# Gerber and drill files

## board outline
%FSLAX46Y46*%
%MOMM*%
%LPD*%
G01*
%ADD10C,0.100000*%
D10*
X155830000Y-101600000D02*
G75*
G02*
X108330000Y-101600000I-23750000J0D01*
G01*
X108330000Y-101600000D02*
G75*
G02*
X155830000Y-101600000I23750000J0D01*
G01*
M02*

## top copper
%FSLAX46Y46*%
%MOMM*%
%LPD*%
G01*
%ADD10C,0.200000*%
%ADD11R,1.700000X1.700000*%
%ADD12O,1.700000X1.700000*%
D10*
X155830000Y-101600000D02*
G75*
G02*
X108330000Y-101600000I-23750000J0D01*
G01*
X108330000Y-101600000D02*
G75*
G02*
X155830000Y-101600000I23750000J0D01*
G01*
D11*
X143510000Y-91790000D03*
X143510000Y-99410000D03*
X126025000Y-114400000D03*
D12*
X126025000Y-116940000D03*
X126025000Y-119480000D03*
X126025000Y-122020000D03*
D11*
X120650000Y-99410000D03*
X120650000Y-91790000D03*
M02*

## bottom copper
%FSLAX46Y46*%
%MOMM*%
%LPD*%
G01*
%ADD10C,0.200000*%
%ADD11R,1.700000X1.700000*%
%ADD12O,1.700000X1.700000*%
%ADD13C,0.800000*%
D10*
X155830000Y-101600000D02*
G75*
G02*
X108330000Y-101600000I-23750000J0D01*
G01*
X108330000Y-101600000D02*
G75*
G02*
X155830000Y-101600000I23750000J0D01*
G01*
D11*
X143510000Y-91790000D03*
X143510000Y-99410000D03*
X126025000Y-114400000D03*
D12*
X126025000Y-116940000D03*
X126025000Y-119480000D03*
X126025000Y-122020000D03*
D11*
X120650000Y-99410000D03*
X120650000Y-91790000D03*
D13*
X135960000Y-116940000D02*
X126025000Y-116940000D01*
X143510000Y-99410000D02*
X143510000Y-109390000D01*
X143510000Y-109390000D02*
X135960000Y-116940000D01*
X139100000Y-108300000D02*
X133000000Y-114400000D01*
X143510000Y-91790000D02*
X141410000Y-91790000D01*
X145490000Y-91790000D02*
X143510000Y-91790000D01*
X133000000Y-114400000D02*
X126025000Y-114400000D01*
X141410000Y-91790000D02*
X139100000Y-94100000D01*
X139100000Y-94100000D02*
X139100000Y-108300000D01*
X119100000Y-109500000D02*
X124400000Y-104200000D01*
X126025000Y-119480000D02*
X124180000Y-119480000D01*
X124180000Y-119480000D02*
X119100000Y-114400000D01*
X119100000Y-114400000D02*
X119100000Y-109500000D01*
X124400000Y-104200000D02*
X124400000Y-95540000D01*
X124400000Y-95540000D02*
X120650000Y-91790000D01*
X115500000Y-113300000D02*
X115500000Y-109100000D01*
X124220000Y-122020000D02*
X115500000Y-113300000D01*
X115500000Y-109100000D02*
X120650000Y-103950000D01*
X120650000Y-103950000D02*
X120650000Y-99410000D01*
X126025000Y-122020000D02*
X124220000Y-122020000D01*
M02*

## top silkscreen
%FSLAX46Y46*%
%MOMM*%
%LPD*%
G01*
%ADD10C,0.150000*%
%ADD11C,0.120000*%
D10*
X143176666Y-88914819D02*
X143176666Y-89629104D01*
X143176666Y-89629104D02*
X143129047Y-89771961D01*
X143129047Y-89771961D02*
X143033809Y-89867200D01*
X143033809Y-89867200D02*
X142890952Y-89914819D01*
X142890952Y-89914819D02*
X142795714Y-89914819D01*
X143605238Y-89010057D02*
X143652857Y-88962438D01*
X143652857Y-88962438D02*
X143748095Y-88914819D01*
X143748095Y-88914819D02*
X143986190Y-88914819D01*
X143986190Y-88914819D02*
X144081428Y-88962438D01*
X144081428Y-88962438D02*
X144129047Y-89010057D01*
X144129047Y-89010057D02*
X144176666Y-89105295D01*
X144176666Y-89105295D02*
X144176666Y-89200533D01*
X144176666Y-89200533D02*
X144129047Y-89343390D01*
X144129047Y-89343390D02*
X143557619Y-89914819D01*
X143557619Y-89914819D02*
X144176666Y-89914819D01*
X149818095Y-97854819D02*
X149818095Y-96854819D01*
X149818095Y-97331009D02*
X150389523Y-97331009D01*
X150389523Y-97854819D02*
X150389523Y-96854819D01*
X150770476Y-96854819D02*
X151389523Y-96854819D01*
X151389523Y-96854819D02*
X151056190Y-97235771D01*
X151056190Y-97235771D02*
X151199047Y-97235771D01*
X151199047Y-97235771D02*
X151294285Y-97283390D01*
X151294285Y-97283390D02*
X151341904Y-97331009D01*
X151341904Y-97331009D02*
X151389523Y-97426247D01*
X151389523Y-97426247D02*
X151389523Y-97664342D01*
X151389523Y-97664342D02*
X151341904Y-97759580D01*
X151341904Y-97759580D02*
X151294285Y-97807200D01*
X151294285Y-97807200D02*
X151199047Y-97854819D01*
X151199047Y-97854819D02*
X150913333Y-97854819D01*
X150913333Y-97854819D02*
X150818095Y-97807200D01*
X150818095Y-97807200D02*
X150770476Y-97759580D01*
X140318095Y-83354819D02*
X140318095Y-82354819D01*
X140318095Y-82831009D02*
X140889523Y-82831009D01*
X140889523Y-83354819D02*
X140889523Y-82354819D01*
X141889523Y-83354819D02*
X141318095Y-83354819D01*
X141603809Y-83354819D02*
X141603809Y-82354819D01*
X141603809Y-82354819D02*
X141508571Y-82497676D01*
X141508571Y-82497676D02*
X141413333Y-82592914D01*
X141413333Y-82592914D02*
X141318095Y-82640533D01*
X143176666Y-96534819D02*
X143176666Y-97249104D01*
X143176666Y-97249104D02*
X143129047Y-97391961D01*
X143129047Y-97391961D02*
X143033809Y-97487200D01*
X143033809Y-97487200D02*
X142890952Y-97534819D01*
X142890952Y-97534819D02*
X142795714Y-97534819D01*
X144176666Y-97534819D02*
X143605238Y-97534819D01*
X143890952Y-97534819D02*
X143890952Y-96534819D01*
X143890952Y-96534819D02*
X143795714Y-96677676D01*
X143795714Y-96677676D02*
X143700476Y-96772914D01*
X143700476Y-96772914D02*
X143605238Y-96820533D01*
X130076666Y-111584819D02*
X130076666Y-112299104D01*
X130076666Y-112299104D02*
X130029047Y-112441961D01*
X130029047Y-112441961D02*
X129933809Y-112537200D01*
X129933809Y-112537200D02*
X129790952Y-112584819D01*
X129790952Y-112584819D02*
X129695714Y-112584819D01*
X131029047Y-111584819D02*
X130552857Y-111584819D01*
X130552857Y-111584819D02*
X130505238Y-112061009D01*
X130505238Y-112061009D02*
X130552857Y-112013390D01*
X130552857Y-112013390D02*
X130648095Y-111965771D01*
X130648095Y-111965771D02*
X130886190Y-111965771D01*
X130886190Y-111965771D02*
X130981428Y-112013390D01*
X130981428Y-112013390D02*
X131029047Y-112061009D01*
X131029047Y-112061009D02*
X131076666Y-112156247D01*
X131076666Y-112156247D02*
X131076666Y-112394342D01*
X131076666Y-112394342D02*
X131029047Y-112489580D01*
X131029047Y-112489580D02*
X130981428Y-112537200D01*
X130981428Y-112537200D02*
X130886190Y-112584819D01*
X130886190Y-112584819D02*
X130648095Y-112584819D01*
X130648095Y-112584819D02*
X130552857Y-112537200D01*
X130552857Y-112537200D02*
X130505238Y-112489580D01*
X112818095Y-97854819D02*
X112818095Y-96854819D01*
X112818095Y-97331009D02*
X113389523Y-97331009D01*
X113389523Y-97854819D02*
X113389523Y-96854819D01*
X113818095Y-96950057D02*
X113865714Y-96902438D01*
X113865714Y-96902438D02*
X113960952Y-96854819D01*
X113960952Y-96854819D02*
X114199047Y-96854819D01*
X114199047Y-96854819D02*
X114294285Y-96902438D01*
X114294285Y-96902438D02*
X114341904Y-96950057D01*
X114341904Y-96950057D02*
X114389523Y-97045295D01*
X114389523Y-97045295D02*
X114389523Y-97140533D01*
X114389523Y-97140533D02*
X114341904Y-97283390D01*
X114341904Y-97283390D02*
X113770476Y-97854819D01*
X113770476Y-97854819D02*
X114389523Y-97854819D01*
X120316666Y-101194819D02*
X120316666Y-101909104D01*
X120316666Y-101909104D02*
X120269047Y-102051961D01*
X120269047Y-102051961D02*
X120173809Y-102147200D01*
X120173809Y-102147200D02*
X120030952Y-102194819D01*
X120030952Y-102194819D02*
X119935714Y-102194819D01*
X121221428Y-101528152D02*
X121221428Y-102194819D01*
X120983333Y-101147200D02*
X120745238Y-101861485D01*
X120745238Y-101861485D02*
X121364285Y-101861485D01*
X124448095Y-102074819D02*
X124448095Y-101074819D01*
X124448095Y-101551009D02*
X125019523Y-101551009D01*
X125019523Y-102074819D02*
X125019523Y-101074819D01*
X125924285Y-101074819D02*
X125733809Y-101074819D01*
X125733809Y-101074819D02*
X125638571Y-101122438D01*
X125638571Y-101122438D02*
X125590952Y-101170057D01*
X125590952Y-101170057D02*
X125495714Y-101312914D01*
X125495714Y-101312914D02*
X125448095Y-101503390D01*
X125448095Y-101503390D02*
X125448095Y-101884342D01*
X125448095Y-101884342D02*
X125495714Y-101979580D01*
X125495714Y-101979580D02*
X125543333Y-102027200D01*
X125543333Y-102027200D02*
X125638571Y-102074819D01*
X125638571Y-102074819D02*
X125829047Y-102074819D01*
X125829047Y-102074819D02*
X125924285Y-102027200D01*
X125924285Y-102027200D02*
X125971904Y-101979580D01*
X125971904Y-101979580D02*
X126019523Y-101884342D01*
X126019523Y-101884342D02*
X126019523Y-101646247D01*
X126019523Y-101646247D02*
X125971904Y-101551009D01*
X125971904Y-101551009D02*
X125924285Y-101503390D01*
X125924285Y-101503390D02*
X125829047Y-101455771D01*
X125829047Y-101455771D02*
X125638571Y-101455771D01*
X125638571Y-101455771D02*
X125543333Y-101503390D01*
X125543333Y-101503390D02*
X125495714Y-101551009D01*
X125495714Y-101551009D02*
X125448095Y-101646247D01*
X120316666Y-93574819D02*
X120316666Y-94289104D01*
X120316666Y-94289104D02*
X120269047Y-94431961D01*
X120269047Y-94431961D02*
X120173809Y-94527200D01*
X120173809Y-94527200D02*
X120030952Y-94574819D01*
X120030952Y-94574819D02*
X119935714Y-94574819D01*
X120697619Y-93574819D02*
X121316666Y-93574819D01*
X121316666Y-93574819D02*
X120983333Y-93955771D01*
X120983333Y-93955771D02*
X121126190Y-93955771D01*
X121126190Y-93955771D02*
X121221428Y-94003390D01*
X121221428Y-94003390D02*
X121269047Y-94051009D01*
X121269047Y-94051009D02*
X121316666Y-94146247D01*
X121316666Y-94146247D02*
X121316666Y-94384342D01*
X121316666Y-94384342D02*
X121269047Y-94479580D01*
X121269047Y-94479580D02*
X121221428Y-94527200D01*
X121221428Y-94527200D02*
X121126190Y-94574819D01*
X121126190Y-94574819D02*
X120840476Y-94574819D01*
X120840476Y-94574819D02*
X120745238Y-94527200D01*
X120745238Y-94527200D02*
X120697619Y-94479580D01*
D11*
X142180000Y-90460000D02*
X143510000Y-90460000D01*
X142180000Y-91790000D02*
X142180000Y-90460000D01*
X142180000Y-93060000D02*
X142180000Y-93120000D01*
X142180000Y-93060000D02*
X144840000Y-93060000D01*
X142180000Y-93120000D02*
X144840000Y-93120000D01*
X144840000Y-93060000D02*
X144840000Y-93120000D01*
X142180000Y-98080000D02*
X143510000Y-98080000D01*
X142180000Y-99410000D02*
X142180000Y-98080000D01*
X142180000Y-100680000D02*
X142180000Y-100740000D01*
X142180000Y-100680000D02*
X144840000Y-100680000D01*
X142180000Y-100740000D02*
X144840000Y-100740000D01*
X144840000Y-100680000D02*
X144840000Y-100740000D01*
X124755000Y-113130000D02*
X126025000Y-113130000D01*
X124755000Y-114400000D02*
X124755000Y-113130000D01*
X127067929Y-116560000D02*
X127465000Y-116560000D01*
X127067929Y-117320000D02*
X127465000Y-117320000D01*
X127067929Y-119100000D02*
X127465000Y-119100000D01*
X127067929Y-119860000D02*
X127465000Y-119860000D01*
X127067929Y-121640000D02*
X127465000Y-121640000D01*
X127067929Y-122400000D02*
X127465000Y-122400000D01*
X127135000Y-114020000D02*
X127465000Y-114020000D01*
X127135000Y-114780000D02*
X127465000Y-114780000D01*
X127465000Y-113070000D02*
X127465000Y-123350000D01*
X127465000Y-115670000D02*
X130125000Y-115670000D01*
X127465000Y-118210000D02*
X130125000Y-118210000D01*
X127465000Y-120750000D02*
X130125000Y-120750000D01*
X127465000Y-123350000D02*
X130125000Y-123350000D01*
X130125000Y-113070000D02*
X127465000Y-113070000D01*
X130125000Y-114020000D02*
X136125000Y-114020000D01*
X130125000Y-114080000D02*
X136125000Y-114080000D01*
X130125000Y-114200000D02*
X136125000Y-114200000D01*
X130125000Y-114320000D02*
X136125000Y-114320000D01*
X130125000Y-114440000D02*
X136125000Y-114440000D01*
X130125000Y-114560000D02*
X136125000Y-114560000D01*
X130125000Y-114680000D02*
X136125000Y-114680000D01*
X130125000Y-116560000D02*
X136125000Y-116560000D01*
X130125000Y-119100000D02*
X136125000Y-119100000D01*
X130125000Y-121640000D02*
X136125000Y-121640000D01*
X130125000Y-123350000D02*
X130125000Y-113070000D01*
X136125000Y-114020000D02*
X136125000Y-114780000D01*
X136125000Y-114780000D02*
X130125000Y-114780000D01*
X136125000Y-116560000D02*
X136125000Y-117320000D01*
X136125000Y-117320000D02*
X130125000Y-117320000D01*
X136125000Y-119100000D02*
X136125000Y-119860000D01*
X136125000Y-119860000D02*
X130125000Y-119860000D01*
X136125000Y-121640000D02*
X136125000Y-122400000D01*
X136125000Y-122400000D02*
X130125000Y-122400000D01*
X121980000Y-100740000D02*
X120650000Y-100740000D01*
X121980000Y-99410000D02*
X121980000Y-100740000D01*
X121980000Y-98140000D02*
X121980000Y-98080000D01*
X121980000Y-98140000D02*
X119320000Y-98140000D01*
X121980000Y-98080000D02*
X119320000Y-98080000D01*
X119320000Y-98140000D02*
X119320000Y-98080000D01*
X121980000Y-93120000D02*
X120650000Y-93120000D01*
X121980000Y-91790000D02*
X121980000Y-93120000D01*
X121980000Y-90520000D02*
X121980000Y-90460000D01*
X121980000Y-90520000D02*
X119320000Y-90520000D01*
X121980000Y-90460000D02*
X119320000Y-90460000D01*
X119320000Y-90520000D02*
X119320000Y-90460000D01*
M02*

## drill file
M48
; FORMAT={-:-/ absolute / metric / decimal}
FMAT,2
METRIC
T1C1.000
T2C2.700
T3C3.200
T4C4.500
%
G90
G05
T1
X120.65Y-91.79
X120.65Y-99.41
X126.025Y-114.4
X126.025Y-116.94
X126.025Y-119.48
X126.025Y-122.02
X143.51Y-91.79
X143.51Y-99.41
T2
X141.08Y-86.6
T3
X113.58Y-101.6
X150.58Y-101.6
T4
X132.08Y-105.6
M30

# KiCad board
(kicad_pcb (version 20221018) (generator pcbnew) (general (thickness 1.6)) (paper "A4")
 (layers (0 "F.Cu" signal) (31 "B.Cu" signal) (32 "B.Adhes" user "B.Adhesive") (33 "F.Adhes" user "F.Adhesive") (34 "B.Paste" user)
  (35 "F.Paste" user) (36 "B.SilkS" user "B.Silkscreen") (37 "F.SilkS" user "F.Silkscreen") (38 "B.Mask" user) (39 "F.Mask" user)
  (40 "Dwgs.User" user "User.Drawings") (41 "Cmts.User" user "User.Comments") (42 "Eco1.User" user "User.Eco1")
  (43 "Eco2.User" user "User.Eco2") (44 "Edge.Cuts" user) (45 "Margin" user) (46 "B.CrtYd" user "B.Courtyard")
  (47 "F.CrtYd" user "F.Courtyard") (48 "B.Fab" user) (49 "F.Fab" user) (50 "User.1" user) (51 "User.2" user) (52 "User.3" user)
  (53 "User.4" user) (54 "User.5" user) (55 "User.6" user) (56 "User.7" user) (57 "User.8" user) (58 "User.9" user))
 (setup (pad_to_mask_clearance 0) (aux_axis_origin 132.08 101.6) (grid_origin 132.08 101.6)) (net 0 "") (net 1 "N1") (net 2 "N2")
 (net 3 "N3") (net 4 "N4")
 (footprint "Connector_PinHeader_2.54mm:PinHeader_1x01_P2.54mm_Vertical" (layer "F.Cu") (at 143.51 91.79)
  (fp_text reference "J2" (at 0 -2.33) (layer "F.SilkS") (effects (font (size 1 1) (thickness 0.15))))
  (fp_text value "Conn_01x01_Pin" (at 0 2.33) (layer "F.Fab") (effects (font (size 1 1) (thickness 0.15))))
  (fp_line (start -1.33 -1.33) (end 0 -1.33) (stroke (width 0.12) (type solid)) (layer "F.SilkS"))
  (fp_line (start -1.33 0) (end -1.33 -1.33) (stroke (width 0.12) (type solid)) (layer "F.SilkS"))
  (fp_line (start -1.33 1.27) (end -1.33 1.33) (stroke (width 0.12) (type solid)) (layer "F.SilkS"))
  (fp_line (start -1.33 1.27) (end 1.33 1.27) (stroke (width 0.12) (type solid)) (layer "F.SilkS"))
  (fp_line (start -1.33 1.33) (end 1.33 1.33) (stroke (width 0.12) (type solid)) (layer "F.SilkS"))
  (fp_line (start 1.33 1.27) (end 1.33 1.33) (stroke (width 0.12) (type solid)) (layer "F.SilkS"))
  (pad "1" thru_hole rect (at 0 0) (size 1.7 1.7) (drill 1) (layers "*.Cu" "*.Mask") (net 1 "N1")))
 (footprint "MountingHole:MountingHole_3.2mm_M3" (layer "F.Cu") (at 150.58 101.6)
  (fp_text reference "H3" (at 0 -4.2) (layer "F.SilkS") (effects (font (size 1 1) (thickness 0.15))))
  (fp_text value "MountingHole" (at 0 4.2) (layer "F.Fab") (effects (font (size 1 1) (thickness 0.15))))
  (pad "" np_thru_hole circle (at 0 0) (size 3.2 3.2) (drill 3.2) (layers "*.Cu" "*.Mask")))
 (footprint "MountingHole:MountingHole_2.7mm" (layer "F.Cu") (at 141.08 86.6)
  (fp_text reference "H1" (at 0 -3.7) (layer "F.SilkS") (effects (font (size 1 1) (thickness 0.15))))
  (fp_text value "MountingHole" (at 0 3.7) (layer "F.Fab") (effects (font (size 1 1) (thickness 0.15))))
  (pad "" np_thru_hole circle (at 0 0) (size 2.7 2.7) (drill 2.7) (layers "*.Cu" "*.Mask")))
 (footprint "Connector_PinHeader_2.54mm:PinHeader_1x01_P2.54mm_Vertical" (layer "F.Cu") (at 143.51 99.41)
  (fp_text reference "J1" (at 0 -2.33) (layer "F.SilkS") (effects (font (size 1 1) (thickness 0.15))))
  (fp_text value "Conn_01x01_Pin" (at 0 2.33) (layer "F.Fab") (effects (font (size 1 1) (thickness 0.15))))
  (fp_line (start -1.33 -1.33) (end 0 -1.33) (stroke (width 0.12) (type solid)) (layer "F.SilkS"))
  (fp_line (start -1.33 0) (end -1.33 -1.33) (stroke (width 0.12) (type solid)) (layer "F.SilkS"))
  (fp_line (start -1.33 1.27) (end -1.33 1.33) (stroke (width 0.12) (type solid)) (layer "F.SilkS"))
  (fp_line (start -1.33 1.27) (end 1.33 1.27) (stroke (width 0.12) (type solid)) (layer "F.SilkS"))
  (fp_line (start -1.33 1.33) (end 1.33 1.33) (stroke (width 0.12) (type solid)) (layer "F.SilkS"))
  (fp_line (start 1.33 1.27) (end 1.33 1.33) (stroke (width 0.12) (type solid)) (layer "F.SilkS"))
  (pad "1" thru_hole rect (at 0 0) (size 1.7 1.7) (drill 1) (layers "*.Cu" "*.Mask") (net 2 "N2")))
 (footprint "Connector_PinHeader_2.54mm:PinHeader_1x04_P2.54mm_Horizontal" (layer "F.Cu") (at 126.025 114.4)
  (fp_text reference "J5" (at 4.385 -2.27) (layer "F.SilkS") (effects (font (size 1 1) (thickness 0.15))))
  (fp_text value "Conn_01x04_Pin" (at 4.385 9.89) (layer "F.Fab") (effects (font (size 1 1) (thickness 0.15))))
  (fp_line (start -1.27 -1.27) (end 0 -1.27) (stroke (width 0.12) (type solid)) (layer "F.SilkS"))
  (fp_line (start -1.27 0) (end -1.27 -1.27) (stroke (width 0.12) (type solid)) (layer "F.SilkS"))
  (fp_line (start 1.042929 2.16) (end 1.44 2.16) (stroke (width 0.12) (type solid)) (layer "F.SilkS"))
  (fp_line (start 1.042929 2.92) (end 1.44 2.92) (stroke (width 0.12) (type solid)) (layer "F.SilkS"))
  (fp_line (start 1.042929 4.7) (end 1.44 4.7) (stroke (width 0.12) (type solid)) (layer "F.SilkS"))
  (fp_line (start 1.042929 5.46) (end 1.44 5.46) (stroke (width 0.12) (type solid)) (layer "F.SilkS"))
  (fp_line (start 1.042929 7.24) (end 1.44 7.24) (stroke (width 0.12) (type solid)) (layer "F.SilkS"))
  (fp_line (start 1.042929 8) (end 1.44 8) (stroke (width 0.12) (type solid)) (layer "F.SilkS"))
  (fp_line (start 1.11 -0.38) (end 1.44 -0.38) (stroke (width 0.12) (type solid)) (layer "F.SilkS"))
  (fp_line (start 1.11 0.38) (end 1.44 0.38) (stroke (width 0.12) (type solid)) (layer "F.SilkS"))
  (fp_line (start 1.44 -1.33) (end 1.44 8.95) (stroke (width 0.12) (type solid)) (layer "F.SilkS"))
  (fp_line (start 1.44 1.27) (end 4.1 1.27) (stroke (width 0.12) (type solid)) (layer "F.SilkS"))
  (fp_line (start 1.44 3.81) (end 4.1 3.81) (stroke (width 0.12) (type solid)) (layer "F.SilkS"))
  (fp_line (start 1.44 6.35) (end 4.1 6.35) (stroke (width 0.12) (type solid)) (layer "F.SilkS"))
  (fp_line (start 1.44 8.95) (end 4.1 8.95) (stroke (width 0.12) (type solid)) (layer "F.SilkS"))
  (fp_line (start 4.1 -1.33) (end 1.44 -1.33) (stroke (width 0.12) (type solid)) (layer "F.SilkS"))
  (fp_line (start 4.1 -0.38) (end 10.1 -0.38) (stroke (width 0.12) (type solid)) (layer "F.SilkS"))
  (fp_line (start 4.1 -0.32) (end 10.1 -0.32) (stroke (width 0.12) (type solid)) (layer "F.SilkS"))
  (fp_line (start 4.1 -0.2) (end 10.1 -0.2) (stroke (width 0.12) (type solid)) (layer "F.SilkS"))
  (fp_line (start 4.1 -0.08) (end 10.1 -0.08) (stroke (width 0.12) (type solid)) (layer "F.SilkS"))
  (fp_line (start 4.1 0.04) (end 10.1 0.04) (stroke (width 0.12) (type solid)) (layer "F.SilkS"))
  (fp_line (start 4.1 0.16) (end 10.1 0.16) (stroke (width 0.12) (type solid)) (layer "F.SilkS"))
  (fp_line (start 4.1 0.28) (end 10.1 0.28) (stroke (width 0.12) (type solid)) (layer "F.SilkS"))
  (fp_line (start 4.1 2.16) (end 10.1 2.16) (stroke (width 0.12) (type solid)) (layer "F.SilkS"))
  (fp_line (start 4.1 4.7) (end 10.1 4.7) (stroke (width 0.12) (type solid)) (layer "F.SilkS"))
  (fp_line (start 4.1 7.24) (end 10.1 7.24) (stroke (width 0.12) (type solid)) (layer "F.SilkS"))
  (fp_line (start 4.1 8.95) (end 4.1 -1.33) (stroke (width 0.12) (type solid)) (layer "F.SilkS"))
  (fp_line (start 10.1 -0.38) (end 10.1 0.38) (stroke (width 0.12) (type solid)) (layer "F.SilkS"))
  (fp_line (start 10.1 0.38) (end 4.1 0.38) (stroke (width 0.12) (type solid)) (layer "F.SilkS"))
  (fp_line (start 10.1 2.16) (end 10.1 2.92) (stroke (width 0.12) (type solid)) (layer "F.SilkS"))
  (fp_line (start 10.1 2.92) (end 4.1 2.92) (stroke (width 0.12) (type solid)) (layer "F.SilkS"))
  (fp_line (start 10.1 4.7) (end 10.1 5.46) (stroke (width 0.12) (type solid)) (layer "F.SilkS"))
  (fp_line (start 10.1 5.46) (end 4.1 5.46) (stroke (width 0.12) (type solid)) (layer "F.SilkS"))
  (fp_line (start 10.1 7.24) (end 10.1 8) (stroke (width 0.12) (type solid)) (layer "F.SilkS"))
  (fp_line (start 10.1 8) (end 4.1 8) (stroke (width 0.12) (type solid)) (layer "F.SilkS"))
  (pad "1" thru_hole rect (at 0 0) (size 1.7 1.7) (drill 1) (layers "*.Cu" "*.Mask") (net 1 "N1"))
  (pad "2" thru_hole oval (at 0 2.54) (size 1.7 1.7) (drill 1) (layers "*.Cu" "*.Mask") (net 2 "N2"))
  (pad "3" thru_hole oval (at 0 5.08) (size 1.7 1.7) (drill 1) (layers "*.Cu" "*.Mask") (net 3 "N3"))
  (pad "4" thru_hole oval (at 0 7.62) (size 1.7 1.7) (drill 1) (layers "*.Cu" "*.Mask") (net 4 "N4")))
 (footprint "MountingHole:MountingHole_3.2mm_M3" (layer "F.Cu") (at 113.58 101.6)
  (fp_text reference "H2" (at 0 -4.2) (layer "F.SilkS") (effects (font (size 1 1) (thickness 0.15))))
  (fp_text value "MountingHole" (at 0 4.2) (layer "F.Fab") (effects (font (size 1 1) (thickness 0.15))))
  (pad "" np_thru_hole circle (at 0 0) (size 3.2 3.2) (drill 3.2) (layers "*.Cu" "*.Mask")))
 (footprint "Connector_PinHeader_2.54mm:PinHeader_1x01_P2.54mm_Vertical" (layer "F.Cu") (at 120.65 99.41 180)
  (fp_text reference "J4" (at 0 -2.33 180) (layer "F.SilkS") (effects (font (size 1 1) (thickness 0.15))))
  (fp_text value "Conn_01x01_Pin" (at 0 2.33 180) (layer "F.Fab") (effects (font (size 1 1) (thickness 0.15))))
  (fp_line (start -1.33 -1.33) (end 0 -1.33) (stroke (width 0.12) (type solid)) (layer "F.SilkS"))
  (fp_line (start -1.33 0) (end -1.33 -1.33) (stroke (width 0.12) (type solid)) (layer "F.SilkS"))
  (fp_line (start -1.33 1.27) (end -1.33 1.33) (stroke (width 0.12) (type solid)) (layer "F.SilkS"))
  (fp_line (start -1.33 1.27) (end 1.33 1.27) (stroke (width 0.12) (type solid)) (layer "F.SilkS"))
  (fp_line (start -1.33 1.33) (end 1.33 1.33) (stroke (width 0.12) (type solid)) (layer "F.SilkS"))
  (fp_line (start 1.33 1.27) (end 1.33 1.33) (stroke (width 0.12) (type solid)) (layer "F.SilkS"))
  (pad "1" thru_hole rect (at 0 0 180) (size 1.7 1.7) (drill 1) (layers "*.Cu" "*.Mask") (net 4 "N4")))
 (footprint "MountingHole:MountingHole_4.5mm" (layer "F.Cu") (at 132.08 105.6)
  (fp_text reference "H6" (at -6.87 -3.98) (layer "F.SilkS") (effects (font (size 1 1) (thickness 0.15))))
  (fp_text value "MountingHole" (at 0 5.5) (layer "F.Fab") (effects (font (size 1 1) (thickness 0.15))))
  (pad "" np_thru_hole circle (at 0 0) (size 4.5 4.5) (drill 4.5) (layers "*.Cu" "*.Mask")))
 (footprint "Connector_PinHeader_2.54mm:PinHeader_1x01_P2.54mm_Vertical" (layer "F.Cu") (at 120.65 91.79 180)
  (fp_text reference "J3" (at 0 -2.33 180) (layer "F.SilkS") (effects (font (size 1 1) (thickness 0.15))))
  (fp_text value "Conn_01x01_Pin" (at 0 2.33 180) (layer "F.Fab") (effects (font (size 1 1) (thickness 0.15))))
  (fp_line (start -1.33 -1.33) (end 0 -1.33) (stroke (width 0.12) (type solid)) (layer "F.SilkS"))
  (fp_line (start -1.33 0) (end -1.33 -1.33) (stroke (width 0.12) (type solid)) (layer "F.SilkS"))
  (fp_line (start -1.33 1.27) (end -1.33 1.33) (stroke (width 0.12) (type solid)) (layer "F.SilkS"))
  (fp_line (start -1.33 1.27) (end 1.33 1.27) (stroke (width 0.12) (type solid)) (layer "F.SilkS"))
  (fp_line (start -1.33 1.33) (end 1.33 1.33) (stroke (width 0.12) (type solid)) (layer "F.SilkS"))
  (fp_line (start 1.33 1.27) (end 1.33 1.33) (stroke (width 0.12) (type solid)) (layer "F.SilkS"))
  (pad "1" thru_hole rect (at 0 0 180) (size 1.7 1.7) (drill 1) (layers "*.Cu" "*.Mask") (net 3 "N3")))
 (gr_circle (center 132.08 101.6) (end 155.83 101.6) (stroke (width 0.2) (type default)) (fill none) (layer "F.Cu"))
 (gr_circle (center 132.08 101.6) (end 155.83 101.6) (stroke (width 0.2) (type default)) (fill none) (layer "B.Cu"))
 (gr_circle (center 132.08 101.6) (end 155.83 101.6) (stroke (width 0.1) (type default)) (fill none) (layer "Edge.Cuts"))
 (segment (start 135.96 116.94) (end 126.025 116.94) (width 0.8) (layer "B.Cu") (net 2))
 (segment (start 143.51 99.41) (end 143.51 109.39) (width 0.8) (layer "B.Cu") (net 2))
 (segment (start 143.51 109.39) (end 135.96 116.94) (width 0.8) (layer "B.Cu") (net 2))
 (segment (start 139.1 108.3) (end 133 114.4) (width 0.8) (layer "B.Cu") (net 1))
 (segment (start 143.51 91.79) (end 141.41 91.79) (width 0.8) (layer "B.Cu") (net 1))
 (segment (start 145.49 91.79) (end 143.51 91.79) (width 0.8) (layer "B.Cu") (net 1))
 (segment (start 133 114.4) (end 126.025 114.4) (width 0.8) (layer "B.Cu") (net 1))
 (segment (start 141.41 91.79) (end 139.1 94.1) (width 0.8) (layer "B.Cu") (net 1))
 (segment (start 139.1 94.1) (end 139.1 108.3) (width 0.8) (layer "B.Cu") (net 1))
 (segment (start 119.1 109.5) (end 124.4 104.2) (width 0.8) (layer "B.Cu") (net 3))
 (segment (start 126.025 119.48) (end 124.18 119.48) (width 0.8) (layer "B.Cu") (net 3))
 (segment (start 124.18 119.48) (end 119.1 114.4) (width 0.8) (layer "B.Cu") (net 3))
 (segment (start 119.1 114.4) (end 119.1 109.5) (width 0.8) (layer "B.Cu") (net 3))
 (segment (start 124.4 104.2) (end 124.4 95.54) (width 0.8) (layer "B.Cu") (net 3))
 (segment (start 124.4 95.54) (end 120.65 91.79) (width 0.8) (layer "B.Cu") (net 3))
 (segment (start 115.5 113.3) (end 115.5 109.1) (width 0.8) (layer "B.Cu") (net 4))
 (segment (start 124.22 122.02) (end 115.5 113.3) (width 0.8) (layer "B.Cu") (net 4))
 (segment (start 115.5 109.1) (end 120.65 103.95) (width 0.8) (layer "B.Cu") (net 4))
 (segment (start 120.65 103.95) (end 120.65 99.41) (width 0.8) (layer "B.Cu") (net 4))
 (segment (start 126.025 122.02) (end 124.22 122.02) (width 0.8) (layer "B.Cu") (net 4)))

